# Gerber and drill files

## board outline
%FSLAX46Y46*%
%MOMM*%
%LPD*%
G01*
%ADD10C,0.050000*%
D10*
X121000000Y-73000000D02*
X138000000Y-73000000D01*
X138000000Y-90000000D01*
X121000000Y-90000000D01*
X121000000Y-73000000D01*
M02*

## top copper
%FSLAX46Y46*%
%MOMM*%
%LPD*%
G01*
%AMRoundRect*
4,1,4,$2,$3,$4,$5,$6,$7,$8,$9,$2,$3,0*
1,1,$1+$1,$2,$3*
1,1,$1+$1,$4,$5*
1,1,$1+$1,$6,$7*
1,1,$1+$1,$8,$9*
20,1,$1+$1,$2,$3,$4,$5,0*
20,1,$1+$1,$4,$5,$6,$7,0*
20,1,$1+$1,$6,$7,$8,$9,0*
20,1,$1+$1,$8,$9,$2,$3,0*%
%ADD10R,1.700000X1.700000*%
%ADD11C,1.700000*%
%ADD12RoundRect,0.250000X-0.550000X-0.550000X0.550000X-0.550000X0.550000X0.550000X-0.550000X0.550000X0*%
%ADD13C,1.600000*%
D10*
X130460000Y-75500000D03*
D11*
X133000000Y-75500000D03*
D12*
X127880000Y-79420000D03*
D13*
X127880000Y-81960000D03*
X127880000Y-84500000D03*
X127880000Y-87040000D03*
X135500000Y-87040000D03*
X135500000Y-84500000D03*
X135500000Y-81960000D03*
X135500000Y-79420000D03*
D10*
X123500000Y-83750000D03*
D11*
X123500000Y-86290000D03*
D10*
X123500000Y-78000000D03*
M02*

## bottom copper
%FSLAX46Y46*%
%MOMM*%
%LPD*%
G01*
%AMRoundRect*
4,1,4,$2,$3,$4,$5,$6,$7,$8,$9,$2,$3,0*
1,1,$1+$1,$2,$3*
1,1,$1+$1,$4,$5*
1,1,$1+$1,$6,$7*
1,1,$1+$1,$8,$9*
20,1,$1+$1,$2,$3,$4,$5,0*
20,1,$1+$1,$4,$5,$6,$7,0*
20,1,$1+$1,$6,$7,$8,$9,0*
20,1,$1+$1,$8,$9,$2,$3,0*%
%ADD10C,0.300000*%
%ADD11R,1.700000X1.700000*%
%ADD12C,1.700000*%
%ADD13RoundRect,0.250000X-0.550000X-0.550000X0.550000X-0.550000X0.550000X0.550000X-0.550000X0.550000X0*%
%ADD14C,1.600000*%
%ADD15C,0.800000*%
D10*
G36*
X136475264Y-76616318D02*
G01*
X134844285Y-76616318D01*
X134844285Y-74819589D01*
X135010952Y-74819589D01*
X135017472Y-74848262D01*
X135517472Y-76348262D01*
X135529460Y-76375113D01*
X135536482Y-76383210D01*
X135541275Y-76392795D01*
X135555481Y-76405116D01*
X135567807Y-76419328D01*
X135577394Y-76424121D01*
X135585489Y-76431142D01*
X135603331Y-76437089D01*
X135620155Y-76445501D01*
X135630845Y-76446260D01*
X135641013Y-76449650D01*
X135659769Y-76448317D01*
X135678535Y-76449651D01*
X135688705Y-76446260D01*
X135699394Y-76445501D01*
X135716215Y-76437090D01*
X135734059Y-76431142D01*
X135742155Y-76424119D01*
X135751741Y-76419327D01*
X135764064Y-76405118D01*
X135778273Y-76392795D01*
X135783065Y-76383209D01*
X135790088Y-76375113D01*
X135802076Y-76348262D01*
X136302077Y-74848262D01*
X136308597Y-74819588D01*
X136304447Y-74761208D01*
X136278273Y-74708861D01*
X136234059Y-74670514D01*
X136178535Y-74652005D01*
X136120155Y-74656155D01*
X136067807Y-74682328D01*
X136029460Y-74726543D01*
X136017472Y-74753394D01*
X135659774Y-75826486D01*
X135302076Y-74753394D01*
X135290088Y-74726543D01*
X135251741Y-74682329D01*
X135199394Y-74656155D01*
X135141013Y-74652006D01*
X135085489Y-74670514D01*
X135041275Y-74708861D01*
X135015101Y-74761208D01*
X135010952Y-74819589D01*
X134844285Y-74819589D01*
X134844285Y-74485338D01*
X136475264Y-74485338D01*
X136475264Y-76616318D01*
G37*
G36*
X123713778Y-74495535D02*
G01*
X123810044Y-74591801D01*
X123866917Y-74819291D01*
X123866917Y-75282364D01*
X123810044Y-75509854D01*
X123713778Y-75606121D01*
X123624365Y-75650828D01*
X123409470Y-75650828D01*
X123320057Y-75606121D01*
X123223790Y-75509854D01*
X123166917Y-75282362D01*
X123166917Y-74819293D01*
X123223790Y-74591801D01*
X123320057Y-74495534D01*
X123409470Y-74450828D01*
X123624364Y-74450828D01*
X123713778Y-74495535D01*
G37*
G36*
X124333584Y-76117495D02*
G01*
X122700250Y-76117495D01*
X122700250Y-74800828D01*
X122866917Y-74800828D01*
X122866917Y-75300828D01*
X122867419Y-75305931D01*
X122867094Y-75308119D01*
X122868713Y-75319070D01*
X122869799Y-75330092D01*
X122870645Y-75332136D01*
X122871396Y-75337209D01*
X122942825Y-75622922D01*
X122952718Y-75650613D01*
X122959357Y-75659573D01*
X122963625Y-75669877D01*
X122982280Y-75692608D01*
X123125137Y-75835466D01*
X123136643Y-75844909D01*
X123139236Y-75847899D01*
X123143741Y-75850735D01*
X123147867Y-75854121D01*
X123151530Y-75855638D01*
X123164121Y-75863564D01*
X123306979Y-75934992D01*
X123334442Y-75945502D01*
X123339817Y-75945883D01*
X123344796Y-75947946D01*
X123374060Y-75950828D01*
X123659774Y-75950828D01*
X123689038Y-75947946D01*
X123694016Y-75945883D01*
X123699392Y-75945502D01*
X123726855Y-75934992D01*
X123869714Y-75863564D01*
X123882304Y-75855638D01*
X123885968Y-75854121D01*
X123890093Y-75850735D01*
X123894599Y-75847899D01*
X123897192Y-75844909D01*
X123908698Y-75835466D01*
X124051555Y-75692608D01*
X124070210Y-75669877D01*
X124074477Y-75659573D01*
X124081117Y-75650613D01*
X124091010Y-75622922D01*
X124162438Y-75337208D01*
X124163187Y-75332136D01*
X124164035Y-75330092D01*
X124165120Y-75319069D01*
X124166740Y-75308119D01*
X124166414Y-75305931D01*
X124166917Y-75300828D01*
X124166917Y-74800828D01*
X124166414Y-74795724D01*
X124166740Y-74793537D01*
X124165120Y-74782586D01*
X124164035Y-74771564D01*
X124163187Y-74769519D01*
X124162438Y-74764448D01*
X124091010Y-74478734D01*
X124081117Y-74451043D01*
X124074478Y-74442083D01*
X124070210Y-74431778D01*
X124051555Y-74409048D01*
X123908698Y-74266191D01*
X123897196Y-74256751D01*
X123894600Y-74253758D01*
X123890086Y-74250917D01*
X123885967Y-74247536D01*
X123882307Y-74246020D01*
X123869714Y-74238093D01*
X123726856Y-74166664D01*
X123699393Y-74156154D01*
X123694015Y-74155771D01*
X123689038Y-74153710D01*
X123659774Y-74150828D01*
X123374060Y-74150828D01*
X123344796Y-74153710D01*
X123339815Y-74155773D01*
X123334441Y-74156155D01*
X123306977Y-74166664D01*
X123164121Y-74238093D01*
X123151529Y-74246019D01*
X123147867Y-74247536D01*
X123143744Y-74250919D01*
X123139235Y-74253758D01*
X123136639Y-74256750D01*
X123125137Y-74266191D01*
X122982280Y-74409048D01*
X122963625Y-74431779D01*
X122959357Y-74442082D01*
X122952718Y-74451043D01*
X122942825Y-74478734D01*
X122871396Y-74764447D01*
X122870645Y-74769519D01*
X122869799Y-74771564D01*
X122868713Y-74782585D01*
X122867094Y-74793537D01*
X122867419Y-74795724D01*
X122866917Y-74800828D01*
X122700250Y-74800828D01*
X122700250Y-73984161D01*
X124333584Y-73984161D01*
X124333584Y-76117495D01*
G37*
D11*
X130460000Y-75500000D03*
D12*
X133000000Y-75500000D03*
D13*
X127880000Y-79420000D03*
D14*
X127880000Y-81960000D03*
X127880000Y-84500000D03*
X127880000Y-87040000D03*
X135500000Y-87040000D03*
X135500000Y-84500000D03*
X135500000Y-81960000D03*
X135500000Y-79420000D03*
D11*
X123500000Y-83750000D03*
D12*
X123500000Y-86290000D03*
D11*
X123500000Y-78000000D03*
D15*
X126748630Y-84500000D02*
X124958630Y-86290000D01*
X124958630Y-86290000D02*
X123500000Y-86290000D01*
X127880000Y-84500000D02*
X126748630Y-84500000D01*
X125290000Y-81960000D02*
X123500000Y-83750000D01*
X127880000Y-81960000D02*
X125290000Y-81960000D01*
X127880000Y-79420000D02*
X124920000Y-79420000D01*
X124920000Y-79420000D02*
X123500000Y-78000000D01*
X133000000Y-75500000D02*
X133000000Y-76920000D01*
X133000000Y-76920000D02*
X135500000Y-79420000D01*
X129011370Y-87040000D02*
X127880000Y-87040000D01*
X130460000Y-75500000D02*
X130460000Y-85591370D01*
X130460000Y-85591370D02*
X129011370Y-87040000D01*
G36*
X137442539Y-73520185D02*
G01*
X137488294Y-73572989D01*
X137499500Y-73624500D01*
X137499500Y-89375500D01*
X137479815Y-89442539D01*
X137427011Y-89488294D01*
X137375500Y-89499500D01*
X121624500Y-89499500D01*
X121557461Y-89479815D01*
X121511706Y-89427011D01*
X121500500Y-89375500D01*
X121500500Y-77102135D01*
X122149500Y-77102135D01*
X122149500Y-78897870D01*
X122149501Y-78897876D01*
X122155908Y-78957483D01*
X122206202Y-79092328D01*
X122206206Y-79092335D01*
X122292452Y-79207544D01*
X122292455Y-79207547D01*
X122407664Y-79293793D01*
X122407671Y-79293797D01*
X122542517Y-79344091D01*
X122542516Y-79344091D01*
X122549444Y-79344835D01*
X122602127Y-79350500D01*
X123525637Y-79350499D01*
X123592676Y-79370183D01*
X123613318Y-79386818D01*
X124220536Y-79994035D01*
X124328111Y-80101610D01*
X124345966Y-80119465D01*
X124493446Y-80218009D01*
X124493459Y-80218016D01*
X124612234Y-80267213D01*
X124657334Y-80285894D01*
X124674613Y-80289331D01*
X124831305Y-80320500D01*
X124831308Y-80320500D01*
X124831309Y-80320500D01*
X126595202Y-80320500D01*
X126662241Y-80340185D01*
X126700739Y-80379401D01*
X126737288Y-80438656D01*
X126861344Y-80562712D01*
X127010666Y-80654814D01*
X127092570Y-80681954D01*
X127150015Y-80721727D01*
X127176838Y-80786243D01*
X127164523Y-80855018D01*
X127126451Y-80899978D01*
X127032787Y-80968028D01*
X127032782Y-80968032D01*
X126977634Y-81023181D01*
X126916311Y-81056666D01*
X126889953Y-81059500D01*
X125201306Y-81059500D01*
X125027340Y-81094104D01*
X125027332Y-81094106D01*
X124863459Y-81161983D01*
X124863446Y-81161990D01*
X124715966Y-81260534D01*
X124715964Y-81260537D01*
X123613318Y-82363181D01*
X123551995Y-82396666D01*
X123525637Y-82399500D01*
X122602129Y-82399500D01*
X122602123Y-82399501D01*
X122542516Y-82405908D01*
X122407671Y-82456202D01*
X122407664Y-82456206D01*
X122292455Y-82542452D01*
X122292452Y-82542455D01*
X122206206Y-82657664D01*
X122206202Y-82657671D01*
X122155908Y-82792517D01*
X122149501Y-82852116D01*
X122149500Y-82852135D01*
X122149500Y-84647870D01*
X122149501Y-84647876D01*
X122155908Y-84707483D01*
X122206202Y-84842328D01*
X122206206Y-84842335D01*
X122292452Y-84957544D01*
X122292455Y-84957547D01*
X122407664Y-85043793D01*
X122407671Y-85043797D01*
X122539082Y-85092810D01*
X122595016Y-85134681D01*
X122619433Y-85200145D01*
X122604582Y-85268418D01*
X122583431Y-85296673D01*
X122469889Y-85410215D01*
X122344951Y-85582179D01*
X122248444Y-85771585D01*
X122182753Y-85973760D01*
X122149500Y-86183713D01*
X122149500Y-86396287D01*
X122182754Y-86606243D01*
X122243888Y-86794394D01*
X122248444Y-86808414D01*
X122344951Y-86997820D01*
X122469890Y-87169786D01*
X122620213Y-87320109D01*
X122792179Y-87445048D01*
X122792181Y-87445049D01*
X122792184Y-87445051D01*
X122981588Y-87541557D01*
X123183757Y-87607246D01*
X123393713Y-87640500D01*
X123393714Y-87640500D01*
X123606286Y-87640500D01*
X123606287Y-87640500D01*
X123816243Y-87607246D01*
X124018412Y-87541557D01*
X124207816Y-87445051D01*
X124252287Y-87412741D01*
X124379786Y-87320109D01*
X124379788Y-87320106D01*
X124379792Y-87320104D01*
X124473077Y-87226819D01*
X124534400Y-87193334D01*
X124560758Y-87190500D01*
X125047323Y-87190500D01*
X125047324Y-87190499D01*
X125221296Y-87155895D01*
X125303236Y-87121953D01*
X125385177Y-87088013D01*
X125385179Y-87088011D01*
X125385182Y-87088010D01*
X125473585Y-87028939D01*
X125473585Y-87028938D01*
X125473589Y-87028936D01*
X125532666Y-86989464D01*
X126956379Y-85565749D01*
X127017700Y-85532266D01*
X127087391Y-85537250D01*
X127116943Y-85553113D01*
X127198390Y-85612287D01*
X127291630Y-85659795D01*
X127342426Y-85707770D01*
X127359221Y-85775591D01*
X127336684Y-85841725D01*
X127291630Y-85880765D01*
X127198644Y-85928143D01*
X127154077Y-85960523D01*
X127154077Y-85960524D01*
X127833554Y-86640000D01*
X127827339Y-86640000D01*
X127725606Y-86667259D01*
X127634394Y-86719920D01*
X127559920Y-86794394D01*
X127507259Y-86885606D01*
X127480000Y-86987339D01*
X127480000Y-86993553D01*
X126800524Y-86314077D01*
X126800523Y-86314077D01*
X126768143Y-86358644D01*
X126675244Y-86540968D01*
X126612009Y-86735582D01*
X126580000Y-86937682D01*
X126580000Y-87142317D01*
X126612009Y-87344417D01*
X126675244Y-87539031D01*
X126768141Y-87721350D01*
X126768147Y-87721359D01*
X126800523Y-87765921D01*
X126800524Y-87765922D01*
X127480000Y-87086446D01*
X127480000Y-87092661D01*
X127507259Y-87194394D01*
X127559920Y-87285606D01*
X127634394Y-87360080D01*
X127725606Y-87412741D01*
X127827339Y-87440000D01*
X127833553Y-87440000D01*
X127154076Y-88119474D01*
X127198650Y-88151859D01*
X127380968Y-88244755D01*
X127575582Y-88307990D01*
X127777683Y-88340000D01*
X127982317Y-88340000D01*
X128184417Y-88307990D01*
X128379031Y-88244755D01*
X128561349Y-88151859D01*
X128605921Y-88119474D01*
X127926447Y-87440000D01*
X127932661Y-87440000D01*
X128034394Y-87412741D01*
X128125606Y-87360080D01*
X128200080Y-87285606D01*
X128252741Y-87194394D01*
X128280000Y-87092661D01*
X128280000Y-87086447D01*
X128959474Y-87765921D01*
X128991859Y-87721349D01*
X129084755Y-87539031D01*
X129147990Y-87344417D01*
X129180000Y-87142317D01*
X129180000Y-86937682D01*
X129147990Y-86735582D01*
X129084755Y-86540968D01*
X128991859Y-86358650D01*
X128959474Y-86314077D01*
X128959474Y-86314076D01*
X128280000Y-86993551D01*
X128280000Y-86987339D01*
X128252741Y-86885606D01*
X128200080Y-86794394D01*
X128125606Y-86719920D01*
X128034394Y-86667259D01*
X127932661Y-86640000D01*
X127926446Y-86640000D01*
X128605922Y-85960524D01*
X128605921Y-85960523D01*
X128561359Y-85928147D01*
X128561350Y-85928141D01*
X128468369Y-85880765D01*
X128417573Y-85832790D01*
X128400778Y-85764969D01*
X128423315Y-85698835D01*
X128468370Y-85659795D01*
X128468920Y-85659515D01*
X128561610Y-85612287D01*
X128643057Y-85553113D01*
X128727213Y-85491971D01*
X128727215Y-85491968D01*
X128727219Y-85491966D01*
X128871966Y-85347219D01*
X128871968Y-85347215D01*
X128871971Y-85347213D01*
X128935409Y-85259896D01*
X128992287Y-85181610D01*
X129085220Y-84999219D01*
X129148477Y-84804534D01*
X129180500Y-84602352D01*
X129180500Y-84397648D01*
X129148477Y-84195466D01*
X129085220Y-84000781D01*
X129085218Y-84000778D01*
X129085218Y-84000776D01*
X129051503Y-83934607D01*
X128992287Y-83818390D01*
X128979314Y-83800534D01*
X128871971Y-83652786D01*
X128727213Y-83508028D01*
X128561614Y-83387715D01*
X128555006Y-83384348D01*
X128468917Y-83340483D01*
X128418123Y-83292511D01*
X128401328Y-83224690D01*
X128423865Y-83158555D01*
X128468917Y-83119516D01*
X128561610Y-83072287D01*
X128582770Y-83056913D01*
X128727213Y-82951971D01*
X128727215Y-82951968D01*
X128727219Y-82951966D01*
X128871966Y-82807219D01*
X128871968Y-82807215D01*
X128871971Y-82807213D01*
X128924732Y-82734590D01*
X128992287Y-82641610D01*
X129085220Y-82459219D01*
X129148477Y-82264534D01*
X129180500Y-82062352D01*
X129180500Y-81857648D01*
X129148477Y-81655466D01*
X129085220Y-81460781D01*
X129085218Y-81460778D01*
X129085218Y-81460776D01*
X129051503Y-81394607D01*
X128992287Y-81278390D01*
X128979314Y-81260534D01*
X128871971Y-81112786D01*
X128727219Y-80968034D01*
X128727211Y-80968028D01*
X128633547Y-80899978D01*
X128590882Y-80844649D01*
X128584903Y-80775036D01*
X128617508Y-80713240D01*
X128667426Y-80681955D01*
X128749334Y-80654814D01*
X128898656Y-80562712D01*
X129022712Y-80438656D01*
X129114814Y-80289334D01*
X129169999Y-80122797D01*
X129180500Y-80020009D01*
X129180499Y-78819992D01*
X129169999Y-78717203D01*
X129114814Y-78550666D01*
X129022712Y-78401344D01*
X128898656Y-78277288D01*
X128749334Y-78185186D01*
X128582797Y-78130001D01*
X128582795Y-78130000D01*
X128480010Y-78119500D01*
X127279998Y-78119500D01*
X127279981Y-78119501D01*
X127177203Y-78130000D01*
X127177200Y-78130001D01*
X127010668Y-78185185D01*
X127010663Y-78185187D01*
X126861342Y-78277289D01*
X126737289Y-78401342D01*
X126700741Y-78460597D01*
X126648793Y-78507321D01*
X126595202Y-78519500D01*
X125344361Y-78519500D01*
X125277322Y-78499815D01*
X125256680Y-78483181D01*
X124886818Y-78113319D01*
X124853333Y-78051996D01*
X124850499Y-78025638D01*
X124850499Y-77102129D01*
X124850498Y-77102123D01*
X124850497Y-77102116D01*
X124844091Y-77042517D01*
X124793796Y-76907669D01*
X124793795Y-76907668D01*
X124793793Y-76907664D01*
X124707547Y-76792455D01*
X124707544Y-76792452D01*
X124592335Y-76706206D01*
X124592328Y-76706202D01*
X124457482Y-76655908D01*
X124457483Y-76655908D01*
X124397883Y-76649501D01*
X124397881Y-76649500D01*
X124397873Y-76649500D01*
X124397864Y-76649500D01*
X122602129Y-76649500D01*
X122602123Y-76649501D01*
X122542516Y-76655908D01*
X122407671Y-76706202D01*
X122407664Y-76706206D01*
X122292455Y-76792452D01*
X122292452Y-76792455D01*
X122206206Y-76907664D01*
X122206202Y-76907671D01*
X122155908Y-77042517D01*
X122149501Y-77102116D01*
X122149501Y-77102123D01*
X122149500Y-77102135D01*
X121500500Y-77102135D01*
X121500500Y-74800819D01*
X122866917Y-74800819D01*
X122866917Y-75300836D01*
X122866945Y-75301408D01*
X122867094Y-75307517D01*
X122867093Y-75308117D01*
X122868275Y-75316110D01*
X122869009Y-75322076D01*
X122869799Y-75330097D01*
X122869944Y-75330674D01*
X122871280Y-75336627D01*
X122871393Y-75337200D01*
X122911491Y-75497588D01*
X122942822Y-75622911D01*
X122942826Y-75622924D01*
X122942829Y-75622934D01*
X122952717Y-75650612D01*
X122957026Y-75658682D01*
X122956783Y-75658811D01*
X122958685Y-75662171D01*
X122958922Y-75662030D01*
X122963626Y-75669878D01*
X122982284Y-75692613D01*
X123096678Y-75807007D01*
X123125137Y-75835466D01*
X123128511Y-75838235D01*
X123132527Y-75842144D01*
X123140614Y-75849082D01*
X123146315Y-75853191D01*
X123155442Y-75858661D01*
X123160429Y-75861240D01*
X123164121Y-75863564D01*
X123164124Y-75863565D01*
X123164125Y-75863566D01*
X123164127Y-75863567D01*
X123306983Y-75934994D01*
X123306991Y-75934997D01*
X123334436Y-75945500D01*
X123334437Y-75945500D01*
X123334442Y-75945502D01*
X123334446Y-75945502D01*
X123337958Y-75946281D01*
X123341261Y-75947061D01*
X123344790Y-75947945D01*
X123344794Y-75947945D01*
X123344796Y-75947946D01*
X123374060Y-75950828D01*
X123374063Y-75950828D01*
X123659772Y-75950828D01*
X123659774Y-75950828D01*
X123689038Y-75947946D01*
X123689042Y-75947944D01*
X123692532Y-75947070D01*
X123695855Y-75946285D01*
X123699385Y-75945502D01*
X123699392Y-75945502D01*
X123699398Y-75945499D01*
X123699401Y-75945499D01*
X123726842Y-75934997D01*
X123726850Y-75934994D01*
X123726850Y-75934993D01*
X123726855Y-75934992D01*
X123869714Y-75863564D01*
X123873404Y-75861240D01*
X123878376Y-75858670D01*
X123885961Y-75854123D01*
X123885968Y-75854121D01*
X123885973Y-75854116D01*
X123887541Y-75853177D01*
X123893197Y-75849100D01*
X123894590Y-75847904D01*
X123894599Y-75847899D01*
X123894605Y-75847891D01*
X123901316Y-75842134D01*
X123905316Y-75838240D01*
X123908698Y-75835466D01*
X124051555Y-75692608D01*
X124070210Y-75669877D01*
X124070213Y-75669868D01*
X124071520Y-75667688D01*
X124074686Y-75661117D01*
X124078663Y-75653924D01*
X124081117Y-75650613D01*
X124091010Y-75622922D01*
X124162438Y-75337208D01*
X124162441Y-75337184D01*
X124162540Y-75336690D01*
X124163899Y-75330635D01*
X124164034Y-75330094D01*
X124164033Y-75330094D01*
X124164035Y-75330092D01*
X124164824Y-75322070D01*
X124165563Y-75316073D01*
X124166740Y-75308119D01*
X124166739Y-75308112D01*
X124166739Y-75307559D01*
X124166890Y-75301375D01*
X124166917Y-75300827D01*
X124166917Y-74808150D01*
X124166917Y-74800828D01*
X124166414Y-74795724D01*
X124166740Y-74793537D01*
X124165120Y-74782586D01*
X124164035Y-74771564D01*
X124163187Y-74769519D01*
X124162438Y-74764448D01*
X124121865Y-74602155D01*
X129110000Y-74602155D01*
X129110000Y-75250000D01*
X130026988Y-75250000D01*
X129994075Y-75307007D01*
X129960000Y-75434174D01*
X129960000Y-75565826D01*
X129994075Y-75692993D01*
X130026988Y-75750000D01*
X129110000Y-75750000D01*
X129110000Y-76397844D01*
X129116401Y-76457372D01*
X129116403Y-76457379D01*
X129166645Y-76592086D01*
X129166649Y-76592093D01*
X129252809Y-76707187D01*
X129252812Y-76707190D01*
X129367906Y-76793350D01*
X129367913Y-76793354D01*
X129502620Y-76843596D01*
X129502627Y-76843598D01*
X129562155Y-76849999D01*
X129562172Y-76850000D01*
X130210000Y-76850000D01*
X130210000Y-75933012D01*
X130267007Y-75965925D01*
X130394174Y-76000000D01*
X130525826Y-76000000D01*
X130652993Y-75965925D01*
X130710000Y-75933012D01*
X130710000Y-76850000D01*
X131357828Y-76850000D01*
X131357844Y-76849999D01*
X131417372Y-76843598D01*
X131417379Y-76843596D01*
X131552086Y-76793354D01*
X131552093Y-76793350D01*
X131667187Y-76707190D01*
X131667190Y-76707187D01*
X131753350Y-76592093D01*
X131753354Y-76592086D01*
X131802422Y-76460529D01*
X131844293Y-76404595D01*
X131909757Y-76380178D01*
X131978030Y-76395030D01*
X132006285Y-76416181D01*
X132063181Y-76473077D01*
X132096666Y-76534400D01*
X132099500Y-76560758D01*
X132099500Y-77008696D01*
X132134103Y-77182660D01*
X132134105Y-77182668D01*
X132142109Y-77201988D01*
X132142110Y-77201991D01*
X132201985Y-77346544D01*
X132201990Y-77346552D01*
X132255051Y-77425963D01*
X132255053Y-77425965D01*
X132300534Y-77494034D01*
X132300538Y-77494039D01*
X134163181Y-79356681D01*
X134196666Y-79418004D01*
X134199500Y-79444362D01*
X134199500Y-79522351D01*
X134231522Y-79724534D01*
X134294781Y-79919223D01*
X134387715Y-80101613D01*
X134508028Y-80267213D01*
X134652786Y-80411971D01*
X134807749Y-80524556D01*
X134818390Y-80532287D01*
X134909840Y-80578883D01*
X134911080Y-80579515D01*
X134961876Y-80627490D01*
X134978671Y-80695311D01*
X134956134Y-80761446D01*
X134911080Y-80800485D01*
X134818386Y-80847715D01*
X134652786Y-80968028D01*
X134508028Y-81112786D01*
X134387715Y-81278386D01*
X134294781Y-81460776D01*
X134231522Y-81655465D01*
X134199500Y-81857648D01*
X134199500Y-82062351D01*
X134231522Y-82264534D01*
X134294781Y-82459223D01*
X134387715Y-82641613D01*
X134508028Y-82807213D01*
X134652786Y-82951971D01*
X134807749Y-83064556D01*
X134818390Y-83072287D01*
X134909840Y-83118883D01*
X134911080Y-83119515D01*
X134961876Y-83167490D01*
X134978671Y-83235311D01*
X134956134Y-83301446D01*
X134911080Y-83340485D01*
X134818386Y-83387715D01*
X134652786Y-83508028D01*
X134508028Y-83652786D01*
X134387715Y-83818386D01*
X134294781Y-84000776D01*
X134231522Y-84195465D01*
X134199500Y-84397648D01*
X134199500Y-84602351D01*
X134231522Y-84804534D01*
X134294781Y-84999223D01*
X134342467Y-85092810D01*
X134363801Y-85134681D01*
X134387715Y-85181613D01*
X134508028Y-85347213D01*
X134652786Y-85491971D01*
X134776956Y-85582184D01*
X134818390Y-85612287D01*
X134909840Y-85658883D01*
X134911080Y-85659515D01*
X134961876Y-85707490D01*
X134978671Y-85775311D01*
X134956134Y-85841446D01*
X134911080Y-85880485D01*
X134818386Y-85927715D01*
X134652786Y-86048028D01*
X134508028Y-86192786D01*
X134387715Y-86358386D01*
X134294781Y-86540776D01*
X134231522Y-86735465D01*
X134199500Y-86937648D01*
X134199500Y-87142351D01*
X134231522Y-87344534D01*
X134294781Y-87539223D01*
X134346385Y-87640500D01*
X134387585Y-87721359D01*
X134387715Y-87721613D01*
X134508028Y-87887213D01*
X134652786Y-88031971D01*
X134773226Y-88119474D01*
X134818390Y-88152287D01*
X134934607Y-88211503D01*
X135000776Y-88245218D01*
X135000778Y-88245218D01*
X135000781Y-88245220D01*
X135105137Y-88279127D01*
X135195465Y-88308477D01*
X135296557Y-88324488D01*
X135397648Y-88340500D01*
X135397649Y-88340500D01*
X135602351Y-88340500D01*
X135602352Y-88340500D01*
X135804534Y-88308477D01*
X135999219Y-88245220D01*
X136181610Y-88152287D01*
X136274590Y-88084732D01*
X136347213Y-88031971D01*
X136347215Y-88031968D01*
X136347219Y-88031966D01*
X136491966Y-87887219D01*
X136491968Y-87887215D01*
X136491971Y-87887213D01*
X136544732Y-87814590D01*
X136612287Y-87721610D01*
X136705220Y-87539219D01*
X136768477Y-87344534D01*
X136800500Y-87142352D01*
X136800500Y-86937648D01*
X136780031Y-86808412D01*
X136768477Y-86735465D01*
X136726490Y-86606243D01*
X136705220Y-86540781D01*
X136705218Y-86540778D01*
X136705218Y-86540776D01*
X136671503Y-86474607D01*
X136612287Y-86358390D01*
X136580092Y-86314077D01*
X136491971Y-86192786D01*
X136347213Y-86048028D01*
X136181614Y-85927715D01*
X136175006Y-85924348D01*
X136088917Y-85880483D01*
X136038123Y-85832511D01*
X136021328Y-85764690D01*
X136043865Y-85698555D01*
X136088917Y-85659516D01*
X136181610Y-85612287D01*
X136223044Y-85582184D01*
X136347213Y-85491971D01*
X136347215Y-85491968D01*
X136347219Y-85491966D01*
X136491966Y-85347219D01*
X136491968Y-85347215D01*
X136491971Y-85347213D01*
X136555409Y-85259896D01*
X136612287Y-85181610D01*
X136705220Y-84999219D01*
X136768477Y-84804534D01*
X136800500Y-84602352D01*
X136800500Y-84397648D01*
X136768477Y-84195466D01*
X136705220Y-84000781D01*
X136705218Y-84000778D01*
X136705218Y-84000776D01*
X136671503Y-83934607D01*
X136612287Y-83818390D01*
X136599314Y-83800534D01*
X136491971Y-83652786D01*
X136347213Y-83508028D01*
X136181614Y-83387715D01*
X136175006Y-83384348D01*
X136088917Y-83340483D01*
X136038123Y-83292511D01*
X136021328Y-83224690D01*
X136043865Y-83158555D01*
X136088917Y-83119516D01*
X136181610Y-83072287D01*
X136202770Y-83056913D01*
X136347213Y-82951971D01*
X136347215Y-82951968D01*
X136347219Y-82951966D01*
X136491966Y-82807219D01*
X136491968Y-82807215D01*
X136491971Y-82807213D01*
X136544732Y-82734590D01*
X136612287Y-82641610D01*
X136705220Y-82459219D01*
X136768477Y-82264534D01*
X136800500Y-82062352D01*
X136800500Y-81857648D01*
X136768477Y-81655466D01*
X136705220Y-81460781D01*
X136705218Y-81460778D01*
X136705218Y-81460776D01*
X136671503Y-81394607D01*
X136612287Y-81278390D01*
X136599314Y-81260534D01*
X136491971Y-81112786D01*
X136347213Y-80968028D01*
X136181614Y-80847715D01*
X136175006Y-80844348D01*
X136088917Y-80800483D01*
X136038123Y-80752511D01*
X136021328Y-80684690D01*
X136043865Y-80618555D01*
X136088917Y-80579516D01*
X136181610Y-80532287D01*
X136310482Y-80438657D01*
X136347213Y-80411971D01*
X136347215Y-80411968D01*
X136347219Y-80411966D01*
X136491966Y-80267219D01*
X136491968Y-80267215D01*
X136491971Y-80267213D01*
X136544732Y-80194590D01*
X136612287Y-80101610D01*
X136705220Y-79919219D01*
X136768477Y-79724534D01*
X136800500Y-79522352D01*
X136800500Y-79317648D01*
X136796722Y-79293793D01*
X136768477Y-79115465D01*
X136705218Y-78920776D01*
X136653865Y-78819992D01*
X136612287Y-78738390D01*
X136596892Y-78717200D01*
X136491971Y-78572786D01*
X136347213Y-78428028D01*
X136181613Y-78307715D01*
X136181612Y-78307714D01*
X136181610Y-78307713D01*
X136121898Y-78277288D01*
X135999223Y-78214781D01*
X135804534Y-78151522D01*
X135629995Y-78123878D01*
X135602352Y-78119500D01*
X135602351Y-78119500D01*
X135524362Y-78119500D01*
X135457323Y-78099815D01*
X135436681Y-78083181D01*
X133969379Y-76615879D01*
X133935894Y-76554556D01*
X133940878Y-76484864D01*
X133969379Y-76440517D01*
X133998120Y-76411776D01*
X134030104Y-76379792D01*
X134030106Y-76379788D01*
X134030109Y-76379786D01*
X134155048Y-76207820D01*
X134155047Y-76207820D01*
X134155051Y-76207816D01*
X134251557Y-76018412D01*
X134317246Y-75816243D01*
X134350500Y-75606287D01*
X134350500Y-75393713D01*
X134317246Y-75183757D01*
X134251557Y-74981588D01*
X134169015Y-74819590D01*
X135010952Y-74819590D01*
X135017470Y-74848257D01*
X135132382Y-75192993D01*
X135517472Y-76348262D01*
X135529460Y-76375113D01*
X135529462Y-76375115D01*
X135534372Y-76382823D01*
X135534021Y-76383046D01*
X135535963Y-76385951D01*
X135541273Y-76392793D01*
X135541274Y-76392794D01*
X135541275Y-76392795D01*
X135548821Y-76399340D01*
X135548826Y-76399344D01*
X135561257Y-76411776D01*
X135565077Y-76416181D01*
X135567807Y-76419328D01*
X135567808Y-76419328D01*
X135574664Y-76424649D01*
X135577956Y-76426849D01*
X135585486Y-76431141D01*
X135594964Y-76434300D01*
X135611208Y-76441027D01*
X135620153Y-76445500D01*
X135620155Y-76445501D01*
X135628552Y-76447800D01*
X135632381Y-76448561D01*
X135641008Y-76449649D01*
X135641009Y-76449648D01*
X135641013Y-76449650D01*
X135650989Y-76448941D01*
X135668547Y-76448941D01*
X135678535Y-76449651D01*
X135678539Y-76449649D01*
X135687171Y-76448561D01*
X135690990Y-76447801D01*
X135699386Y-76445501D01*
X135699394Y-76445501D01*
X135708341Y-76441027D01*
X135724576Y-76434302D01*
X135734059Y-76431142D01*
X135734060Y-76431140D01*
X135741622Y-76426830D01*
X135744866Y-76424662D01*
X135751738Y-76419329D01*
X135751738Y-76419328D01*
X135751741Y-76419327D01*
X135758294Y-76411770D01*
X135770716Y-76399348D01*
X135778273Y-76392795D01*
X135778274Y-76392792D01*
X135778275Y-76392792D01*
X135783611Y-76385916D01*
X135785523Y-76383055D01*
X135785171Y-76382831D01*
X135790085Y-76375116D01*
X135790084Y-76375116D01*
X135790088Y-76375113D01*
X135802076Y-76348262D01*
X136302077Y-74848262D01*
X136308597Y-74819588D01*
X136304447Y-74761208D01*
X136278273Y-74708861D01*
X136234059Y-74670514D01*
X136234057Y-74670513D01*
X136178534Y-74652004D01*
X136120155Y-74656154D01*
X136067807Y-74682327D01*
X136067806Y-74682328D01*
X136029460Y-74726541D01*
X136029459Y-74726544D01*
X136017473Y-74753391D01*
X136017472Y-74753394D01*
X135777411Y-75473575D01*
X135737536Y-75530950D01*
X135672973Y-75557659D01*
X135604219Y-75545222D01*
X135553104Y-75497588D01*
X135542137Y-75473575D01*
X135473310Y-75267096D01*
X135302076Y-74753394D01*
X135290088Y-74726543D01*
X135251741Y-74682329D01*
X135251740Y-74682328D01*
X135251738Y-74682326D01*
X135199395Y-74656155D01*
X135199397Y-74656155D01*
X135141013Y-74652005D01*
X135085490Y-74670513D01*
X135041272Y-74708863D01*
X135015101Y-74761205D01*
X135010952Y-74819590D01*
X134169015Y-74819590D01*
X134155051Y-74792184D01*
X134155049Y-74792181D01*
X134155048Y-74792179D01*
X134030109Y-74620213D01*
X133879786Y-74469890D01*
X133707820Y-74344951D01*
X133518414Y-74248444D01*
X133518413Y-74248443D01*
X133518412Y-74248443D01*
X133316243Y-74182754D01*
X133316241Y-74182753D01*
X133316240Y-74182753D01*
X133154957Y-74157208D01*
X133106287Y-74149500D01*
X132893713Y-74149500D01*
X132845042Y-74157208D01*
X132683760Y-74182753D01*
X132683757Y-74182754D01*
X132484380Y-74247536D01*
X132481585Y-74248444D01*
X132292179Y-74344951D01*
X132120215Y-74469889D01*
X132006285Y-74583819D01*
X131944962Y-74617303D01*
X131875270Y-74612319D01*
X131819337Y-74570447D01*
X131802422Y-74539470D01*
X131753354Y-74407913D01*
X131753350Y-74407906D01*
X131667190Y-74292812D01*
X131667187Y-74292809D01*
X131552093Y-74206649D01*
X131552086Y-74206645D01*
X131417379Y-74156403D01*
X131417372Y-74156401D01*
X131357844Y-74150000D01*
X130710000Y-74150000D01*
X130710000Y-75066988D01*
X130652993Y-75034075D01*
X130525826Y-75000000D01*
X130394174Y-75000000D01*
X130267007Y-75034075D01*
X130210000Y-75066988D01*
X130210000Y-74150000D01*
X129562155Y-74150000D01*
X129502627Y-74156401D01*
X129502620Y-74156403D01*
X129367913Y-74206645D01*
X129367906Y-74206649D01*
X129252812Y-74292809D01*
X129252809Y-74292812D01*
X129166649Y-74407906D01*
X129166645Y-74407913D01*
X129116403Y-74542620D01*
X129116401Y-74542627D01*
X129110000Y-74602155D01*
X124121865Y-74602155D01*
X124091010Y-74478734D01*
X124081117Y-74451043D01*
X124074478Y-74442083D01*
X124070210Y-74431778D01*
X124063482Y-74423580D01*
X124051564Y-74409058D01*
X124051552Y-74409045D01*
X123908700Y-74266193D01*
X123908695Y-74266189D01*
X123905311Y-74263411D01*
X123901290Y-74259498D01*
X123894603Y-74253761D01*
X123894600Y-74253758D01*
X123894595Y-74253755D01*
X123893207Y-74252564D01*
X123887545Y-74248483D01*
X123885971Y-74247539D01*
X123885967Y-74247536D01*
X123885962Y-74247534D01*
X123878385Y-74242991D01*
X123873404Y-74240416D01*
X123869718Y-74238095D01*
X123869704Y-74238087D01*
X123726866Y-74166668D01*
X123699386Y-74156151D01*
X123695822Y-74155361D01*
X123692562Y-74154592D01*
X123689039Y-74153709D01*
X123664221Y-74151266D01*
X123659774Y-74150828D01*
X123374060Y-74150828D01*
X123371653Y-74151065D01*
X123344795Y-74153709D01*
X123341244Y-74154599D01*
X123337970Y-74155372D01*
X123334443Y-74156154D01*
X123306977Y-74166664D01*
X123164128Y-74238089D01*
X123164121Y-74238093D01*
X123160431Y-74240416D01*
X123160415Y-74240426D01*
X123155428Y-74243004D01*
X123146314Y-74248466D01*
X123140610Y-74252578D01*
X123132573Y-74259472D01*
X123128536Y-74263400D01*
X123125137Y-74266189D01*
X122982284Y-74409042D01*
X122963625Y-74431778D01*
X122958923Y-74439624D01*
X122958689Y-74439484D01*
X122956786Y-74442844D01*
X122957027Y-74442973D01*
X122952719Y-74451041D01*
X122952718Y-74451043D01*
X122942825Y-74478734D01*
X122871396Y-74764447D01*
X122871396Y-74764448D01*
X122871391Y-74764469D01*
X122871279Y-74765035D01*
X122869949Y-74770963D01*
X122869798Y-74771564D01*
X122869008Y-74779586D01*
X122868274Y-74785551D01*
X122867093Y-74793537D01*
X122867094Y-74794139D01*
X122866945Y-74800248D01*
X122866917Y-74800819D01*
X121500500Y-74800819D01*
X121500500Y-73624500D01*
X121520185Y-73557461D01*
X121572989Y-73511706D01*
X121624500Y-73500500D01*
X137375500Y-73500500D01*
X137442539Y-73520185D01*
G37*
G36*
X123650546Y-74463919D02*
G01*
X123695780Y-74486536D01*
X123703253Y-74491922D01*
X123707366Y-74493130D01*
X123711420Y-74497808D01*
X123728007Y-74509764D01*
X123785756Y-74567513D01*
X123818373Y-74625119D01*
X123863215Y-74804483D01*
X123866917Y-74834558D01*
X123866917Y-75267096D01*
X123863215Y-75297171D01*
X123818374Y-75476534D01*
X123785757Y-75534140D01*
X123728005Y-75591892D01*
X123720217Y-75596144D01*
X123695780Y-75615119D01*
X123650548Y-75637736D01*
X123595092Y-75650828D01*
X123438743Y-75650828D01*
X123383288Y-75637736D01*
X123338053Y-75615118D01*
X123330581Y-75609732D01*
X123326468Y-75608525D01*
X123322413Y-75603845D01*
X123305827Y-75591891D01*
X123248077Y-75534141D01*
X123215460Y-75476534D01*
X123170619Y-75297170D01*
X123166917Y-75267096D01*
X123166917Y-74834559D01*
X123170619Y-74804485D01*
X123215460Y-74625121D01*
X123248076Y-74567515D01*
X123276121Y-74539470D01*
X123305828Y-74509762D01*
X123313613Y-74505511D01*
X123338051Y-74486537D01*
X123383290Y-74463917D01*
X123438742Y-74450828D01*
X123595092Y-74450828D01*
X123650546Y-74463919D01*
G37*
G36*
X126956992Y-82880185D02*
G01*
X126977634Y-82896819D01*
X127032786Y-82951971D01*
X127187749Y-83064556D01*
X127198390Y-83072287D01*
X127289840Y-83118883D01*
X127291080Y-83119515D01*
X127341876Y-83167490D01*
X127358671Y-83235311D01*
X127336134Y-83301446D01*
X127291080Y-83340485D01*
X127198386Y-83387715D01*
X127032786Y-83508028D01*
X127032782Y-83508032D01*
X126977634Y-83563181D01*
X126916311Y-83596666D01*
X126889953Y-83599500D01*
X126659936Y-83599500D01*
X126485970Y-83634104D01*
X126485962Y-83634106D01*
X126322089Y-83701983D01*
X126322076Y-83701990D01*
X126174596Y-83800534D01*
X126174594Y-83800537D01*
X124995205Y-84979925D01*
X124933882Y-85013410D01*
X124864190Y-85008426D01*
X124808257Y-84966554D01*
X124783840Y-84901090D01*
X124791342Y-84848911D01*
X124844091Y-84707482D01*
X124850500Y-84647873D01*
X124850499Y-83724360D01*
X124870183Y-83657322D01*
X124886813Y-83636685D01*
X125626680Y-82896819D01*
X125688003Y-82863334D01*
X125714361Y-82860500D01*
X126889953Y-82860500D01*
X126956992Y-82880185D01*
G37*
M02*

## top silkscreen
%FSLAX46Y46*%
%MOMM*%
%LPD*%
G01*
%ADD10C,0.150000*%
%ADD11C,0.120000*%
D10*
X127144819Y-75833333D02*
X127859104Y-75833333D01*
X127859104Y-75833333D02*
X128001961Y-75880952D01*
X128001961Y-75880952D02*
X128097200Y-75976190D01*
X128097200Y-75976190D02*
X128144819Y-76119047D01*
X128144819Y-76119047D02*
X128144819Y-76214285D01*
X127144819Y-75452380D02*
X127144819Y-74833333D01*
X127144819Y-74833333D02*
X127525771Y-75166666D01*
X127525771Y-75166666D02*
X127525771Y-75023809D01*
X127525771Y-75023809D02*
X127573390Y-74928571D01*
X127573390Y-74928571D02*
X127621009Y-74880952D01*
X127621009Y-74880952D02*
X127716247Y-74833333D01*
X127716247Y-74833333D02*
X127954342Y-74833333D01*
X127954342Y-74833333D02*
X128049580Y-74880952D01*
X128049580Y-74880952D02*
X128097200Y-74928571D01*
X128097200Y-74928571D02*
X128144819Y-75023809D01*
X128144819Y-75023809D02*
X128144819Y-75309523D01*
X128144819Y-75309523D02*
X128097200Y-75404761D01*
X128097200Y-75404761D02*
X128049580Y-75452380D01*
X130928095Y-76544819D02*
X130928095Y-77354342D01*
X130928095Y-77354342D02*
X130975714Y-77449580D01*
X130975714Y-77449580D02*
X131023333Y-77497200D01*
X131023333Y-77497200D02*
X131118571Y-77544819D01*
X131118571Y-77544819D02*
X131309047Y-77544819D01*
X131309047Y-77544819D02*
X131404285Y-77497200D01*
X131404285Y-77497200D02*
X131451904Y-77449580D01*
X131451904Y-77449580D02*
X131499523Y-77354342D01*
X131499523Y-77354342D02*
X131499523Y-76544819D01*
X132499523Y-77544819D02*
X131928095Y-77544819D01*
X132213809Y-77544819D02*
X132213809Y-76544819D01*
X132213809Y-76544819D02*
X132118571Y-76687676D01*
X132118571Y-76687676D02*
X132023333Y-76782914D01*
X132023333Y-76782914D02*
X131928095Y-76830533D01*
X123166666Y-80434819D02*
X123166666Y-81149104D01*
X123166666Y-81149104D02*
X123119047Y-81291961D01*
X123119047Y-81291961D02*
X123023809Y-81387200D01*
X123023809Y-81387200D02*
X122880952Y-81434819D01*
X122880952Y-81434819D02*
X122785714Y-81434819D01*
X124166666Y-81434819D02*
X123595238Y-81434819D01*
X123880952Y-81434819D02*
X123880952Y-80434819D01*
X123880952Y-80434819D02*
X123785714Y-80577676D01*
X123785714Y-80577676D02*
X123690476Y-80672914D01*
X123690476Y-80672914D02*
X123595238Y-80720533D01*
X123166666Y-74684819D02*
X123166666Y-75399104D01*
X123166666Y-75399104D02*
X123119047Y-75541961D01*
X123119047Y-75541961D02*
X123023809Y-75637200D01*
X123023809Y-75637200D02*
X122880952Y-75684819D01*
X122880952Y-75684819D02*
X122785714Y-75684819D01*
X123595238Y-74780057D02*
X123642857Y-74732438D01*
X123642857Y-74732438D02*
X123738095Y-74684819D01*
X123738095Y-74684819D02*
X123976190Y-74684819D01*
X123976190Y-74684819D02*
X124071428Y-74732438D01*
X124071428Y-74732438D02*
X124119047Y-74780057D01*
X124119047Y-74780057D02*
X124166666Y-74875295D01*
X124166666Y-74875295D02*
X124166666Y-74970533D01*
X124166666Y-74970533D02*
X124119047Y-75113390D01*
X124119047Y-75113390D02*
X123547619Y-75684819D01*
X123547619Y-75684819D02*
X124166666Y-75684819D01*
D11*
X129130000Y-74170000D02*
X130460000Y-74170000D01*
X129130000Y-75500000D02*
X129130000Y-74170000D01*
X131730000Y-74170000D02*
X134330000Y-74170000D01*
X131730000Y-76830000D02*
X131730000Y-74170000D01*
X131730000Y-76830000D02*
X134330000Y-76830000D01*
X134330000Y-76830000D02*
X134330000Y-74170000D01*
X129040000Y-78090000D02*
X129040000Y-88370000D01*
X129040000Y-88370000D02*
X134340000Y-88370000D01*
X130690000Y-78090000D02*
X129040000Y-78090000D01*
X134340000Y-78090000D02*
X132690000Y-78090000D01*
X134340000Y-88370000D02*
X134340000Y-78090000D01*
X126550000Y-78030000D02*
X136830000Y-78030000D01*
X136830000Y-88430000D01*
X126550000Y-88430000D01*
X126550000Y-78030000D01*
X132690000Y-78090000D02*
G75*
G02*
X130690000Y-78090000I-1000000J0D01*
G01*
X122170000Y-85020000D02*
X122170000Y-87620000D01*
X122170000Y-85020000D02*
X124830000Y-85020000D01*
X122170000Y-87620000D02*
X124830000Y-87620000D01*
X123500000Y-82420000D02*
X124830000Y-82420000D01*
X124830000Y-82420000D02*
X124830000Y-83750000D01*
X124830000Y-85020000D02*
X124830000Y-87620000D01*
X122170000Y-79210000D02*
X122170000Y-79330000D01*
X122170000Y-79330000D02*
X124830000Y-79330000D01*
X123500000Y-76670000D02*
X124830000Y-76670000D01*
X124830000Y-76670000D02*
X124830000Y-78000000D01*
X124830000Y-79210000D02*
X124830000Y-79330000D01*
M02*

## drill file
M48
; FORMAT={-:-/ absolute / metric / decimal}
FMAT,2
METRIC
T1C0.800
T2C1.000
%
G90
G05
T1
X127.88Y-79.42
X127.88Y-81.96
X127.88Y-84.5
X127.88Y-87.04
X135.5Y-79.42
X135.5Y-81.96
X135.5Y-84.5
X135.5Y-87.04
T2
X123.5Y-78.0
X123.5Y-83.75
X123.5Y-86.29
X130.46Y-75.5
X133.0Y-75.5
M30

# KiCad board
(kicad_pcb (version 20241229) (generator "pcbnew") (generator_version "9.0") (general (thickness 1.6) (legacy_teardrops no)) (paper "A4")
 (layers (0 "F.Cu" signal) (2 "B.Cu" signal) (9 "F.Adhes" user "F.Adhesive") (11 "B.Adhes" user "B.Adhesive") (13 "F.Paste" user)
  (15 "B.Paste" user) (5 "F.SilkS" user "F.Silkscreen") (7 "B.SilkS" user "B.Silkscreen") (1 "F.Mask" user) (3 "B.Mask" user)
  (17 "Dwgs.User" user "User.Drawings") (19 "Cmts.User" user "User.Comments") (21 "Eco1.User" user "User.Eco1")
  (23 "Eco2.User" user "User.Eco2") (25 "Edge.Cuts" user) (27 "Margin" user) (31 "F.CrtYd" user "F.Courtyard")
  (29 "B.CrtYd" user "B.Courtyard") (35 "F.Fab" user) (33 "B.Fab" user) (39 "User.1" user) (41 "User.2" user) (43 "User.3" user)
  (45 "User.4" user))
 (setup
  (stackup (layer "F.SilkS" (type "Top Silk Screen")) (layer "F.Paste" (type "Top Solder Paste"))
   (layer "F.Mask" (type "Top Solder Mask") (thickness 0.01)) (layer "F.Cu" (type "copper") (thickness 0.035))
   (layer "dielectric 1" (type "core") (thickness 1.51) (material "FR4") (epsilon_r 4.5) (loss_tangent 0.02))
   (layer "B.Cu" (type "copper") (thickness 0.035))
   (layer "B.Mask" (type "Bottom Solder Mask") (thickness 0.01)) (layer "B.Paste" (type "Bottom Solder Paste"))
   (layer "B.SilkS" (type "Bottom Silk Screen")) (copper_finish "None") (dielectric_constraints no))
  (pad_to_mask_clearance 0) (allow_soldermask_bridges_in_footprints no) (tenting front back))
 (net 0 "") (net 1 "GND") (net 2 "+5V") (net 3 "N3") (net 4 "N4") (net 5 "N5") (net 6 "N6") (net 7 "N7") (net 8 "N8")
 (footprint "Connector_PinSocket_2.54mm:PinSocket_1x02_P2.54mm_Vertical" (layer "F.Cu") (at 130.46 75.5 90)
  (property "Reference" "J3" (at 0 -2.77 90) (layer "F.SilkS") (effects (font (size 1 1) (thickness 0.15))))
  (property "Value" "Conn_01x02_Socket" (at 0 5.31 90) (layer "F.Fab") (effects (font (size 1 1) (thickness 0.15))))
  (fp_line (start 1.33 -1.33) (end 1.33 0) (stroke (width 0.12) (type solid)) (layer "F.SilkS"))
  (fp_line (start 0 -1.33) (end 1.33 -1.33) (stroke (width 0.12) (type solid)) (layer "F.SilkS"))
  (fp_line (start 1.33 1.27) (end 1.33 3.87) (stroke (width 0.12) (type solid)) (layer "F.SilkS"))
  (fp_line (start -1.33 1.27) (end 1.33 1.27) (stroke (width 0.12) (type solid)) (layer "F.SilkS"))
  (fp_line (start -1.33 1.27) (end -1.33 3.87) (stroke (width 0.12) (type solid)) (layer "F.SilkS"))
  (fp_line (start -1.33 3.87) (end 1.33 3.87) (stroke (width 0.12) (type solid)) (layer "F.SilkS"))
  (pad "1" thru_hole rect (at 0 0 90) (size 1.7 1.7) (drill 1) (layers "*.Cu" "*.Mask") (remove_unused_layers no) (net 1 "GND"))
  (pad "2" thru_hole circle (at 0 2.54 90) (size 1.7 1.7) (drill 1) (layers "*.Cu" "*.Mask") (remove_unused_layers no) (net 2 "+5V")))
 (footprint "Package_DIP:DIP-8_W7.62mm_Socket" (layer "F.Cu") (at 127.88 79.42)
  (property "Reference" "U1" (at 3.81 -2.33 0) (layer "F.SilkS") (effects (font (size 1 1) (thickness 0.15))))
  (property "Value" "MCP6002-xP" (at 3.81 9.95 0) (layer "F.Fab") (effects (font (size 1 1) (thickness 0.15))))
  (fp_line (start 1.16 -1.33) (end 1.16 8.95) (stroke (width 0.12) (type solid)) (layer "F.SilkS"))
  (fp_line (start 1.16 8.95) (end 6.46 8.95) (stroke (width 0.12) (type solid)) (layer "F.SilkS"))
  (fp_line (start 2.81 -1.33) (end 1.16 -1.33) (stroke (width 0.12) (type solid)) (layer "F.SilkS"))
  (fp_line (start 6.46 -1.33) (end 4.81 -1.33) (stroke (width 0.12) (type solid)) (layer "F.SilkS"))
  (fp_line (start 6.46 8.95) (end 6.46 -1.33) (stroke (width 0.12) (type solid)) (layer "F.SilkS"))
  (fp_rect (start -1.33 -1.39) (end 8.95 9.01) (stroke (width 0.12) (type solid)) (fill no) (layer "F.SilkS"))
  (fp_arc (start 4.81 -1.33) (mid 3.81 -0.33) (end 2.81 -1.33) (stroke (width 0.12) (type solid)) (layer "F.SilkS"))
  (pad "1" thru_hole roundrect (at 0 0) (size 1.6 1.6) (drill 0.8) (layers "*.Cu" "*.Mask") (remove_unused_layers no)
   (roundrect_rratio 0.15625) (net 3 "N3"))
  (pad "2" thru_hole circle (at 0 2.54) (size 1.6 1.6) (drill 0.8) (layers "*.Cu" "*.Mask") (remove_unused_layers no) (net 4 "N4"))
  (pad "3" thru_hole circle (at 0 5.08) (size 1.6 1.6) (drill 0.8) (layers "*.Cu" "*.Mask") (remove_unused_layers no) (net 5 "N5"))
  (pad "4" thru_hole circle (at 0 7.62) (size 1.6 1.6) (drill 0.8) (layers "*.Cu" "*.Mask") (remove_unused_layers no) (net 1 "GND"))
  (pad "5" thru_hole circle (at 7.62 7.62) (size 1.6 1.6) (drill 0.8) (layers "*.Cu" "*.Mask") (remove_unused_layers no) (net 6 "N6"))
  (pad "6" thru_hole circle (at 7.62 5.08) (size 1.6 1.6) (drill 0.8) (layers "*.Cu" "*.Mask") (remove_unused_layers no) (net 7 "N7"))
  (pad "7" thru_hole circle (at 7.62 2.54) (size 1.6 1.6) (drill 0.8) (layers "*.Cu" "*.Mask") (remove_unused_layers no) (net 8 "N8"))
  (pad "8" thru_hole circle (at 7.62 0) (size 1.6 1.6) (drill 0.8) (layers "*.Cu" "*.Mask") (remove_unused_layers no) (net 2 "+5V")))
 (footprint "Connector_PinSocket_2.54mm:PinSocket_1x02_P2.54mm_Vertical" (layer "F.Cu") (at 123.5 83.75)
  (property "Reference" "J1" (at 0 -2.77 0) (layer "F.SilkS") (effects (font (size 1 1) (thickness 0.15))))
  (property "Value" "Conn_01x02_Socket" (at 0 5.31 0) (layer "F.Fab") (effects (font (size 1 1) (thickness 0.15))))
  (fp_line (start -1.33 1.27) (end -1.33 3.87) (stroke (width 0.12) (type solid)) (layer "F.SilkS"))
  (fp_line (start -1.33 1.27) (end 1.33 1.27) (stroke (width 0.12) (type solid)) (layer "F.SilkS"))
  (fp_line (start -1.33 3.87) (end 1.33 3.87) (stroke (width 0.12) (type solid)) (layer "F.SilkS"))
  (fp_line (start 0 -1.33) (end 1.33 -1.33) (stroke (width 0.12) (type solid)) (layer "F.SilkS"))
  (fp_line (start 1.33 -1.33) (end 1.33 0) (stroke (width 0.12) (type solid)) (layer "F.SilkS"))
  (fp_line (start 1.33 1.27) (end 1.33 3.87) (stroke (width 0.12) (type solid)) (layer "F.SilkS"))
  (pad "1" thru_hole rect (at 0 0) (size 1.7 1.7) (drill 1) (layers "*.Cu" "*.Mask") (remove_unused_layers no) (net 4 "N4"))
  (pad "2" thru_hole circle (at 0 2.54) (size 1.7 1.7) (drill 1) (layers "*.Cu" "*.Mask") (remove_unused_layers no) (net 5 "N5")))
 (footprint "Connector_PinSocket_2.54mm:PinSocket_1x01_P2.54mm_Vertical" (layer "F.Cu") (at 123.5 78)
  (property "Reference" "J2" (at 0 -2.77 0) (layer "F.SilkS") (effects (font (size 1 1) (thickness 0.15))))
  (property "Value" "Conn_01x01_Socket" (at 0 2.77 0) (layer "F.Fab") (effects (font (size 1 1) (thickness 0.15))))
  (fp_line (start -1.33 1.21) (end -1.33 1.33) (stroke (width 0.12) (type solid)) (layer "F.SilkS"))
  (fp_line (start -1.33 1.33) (end 1.33 1.33) (stroke (width 0.12) (type solid)) (layer "F.SilkS"))
  (fp_line (start 0 -1.33) (end 1.33 -1.33) (stroke (width 0.12) (type solid)) (layer "F.SilkS"))
  (fp_line (start 1.33 -1.33) (end 1.33 0) (stroke (width 0.12) (type solid)) (layer "F.SilkS"))
  (fp_line (start 1.33 1.21) (end 1.33 1.33) (stroke (width 0.12) (type solid)) (layer "F.SilkS"))
  (pad "1" thru_hole rect (at 0 0) (size 1.7 1.7) (drill 1) (layers "*.Cu" "*.Mask") (remove_unused_layers no) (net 3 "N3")))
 (gr_rect (start 121 73) (end 138 90) (stroke (width 0.05) (type default)) (fill no) (layer "Edge.Cuts"))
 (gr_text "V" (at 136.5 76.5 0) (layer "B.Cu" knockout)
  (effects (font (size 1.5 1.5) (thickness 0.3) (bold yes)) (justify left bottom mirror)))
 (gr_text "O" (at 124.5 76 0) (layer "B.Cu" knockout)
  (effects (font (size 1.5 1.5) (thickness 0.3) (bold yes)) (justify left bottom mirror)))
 (segment (start 126.74863 84.5) (end 124.95863 86.29) (width 0.8) (layer "B.Cu") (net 5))
 (segment (start 124.95863 86.29) (end 123.5 86.29) (width 0.8) (layer "B.Cu") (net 5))
 (segment (start 127.88 84.5) (end 126.74863 84.5) (width 0.8) (layer "B.Cu") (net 5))
 (segment (start 125.29 81.96) (end 123.5 83.75) (width 0.8) (layer "B.Cu") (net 4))
 (segment (start 127.88 81.96) (end 125.29 81.96) (width 0.8) (layer "B.Cu") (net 4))
 (segment (start 127.88 79.42) (end 124.92 79.42) (width 0.8) (layer "B.Cu") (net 3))
 (segment (start 124.92 79.42) (end 123.5 78) (width 0.8) (layer "B.Cu") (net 3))
 (segment (start 133 75.5) (end 133 76.92) (width 0.8) (layer "B.Cu") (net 2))
 (segment (start 133 76.92) (end 135.5 79.42) (width 0.8) (layer "B.Cu") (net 2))
 (segment (start 129.01137 87.04) (end 127.88 87.04) (width 0.8) (layer "B.Cu") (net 1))
 (segment (start 130.46 75.5) (end 130.46 85.59137) (width 0.8) (layer "B.Cu") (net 1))
 (segment (start 130.46 85.59137) (end 129.01137 87.04) (width 0.8) (layer "B.Cu") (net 1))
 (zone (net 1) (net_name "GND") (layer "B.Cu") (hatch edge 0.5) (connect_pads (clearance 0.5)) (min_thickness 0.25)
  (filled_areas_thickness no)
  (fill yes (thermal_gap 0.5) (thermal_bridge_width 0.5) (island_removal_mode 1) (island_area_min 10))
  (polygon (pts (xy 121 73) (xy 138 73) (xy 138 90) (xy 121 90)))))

